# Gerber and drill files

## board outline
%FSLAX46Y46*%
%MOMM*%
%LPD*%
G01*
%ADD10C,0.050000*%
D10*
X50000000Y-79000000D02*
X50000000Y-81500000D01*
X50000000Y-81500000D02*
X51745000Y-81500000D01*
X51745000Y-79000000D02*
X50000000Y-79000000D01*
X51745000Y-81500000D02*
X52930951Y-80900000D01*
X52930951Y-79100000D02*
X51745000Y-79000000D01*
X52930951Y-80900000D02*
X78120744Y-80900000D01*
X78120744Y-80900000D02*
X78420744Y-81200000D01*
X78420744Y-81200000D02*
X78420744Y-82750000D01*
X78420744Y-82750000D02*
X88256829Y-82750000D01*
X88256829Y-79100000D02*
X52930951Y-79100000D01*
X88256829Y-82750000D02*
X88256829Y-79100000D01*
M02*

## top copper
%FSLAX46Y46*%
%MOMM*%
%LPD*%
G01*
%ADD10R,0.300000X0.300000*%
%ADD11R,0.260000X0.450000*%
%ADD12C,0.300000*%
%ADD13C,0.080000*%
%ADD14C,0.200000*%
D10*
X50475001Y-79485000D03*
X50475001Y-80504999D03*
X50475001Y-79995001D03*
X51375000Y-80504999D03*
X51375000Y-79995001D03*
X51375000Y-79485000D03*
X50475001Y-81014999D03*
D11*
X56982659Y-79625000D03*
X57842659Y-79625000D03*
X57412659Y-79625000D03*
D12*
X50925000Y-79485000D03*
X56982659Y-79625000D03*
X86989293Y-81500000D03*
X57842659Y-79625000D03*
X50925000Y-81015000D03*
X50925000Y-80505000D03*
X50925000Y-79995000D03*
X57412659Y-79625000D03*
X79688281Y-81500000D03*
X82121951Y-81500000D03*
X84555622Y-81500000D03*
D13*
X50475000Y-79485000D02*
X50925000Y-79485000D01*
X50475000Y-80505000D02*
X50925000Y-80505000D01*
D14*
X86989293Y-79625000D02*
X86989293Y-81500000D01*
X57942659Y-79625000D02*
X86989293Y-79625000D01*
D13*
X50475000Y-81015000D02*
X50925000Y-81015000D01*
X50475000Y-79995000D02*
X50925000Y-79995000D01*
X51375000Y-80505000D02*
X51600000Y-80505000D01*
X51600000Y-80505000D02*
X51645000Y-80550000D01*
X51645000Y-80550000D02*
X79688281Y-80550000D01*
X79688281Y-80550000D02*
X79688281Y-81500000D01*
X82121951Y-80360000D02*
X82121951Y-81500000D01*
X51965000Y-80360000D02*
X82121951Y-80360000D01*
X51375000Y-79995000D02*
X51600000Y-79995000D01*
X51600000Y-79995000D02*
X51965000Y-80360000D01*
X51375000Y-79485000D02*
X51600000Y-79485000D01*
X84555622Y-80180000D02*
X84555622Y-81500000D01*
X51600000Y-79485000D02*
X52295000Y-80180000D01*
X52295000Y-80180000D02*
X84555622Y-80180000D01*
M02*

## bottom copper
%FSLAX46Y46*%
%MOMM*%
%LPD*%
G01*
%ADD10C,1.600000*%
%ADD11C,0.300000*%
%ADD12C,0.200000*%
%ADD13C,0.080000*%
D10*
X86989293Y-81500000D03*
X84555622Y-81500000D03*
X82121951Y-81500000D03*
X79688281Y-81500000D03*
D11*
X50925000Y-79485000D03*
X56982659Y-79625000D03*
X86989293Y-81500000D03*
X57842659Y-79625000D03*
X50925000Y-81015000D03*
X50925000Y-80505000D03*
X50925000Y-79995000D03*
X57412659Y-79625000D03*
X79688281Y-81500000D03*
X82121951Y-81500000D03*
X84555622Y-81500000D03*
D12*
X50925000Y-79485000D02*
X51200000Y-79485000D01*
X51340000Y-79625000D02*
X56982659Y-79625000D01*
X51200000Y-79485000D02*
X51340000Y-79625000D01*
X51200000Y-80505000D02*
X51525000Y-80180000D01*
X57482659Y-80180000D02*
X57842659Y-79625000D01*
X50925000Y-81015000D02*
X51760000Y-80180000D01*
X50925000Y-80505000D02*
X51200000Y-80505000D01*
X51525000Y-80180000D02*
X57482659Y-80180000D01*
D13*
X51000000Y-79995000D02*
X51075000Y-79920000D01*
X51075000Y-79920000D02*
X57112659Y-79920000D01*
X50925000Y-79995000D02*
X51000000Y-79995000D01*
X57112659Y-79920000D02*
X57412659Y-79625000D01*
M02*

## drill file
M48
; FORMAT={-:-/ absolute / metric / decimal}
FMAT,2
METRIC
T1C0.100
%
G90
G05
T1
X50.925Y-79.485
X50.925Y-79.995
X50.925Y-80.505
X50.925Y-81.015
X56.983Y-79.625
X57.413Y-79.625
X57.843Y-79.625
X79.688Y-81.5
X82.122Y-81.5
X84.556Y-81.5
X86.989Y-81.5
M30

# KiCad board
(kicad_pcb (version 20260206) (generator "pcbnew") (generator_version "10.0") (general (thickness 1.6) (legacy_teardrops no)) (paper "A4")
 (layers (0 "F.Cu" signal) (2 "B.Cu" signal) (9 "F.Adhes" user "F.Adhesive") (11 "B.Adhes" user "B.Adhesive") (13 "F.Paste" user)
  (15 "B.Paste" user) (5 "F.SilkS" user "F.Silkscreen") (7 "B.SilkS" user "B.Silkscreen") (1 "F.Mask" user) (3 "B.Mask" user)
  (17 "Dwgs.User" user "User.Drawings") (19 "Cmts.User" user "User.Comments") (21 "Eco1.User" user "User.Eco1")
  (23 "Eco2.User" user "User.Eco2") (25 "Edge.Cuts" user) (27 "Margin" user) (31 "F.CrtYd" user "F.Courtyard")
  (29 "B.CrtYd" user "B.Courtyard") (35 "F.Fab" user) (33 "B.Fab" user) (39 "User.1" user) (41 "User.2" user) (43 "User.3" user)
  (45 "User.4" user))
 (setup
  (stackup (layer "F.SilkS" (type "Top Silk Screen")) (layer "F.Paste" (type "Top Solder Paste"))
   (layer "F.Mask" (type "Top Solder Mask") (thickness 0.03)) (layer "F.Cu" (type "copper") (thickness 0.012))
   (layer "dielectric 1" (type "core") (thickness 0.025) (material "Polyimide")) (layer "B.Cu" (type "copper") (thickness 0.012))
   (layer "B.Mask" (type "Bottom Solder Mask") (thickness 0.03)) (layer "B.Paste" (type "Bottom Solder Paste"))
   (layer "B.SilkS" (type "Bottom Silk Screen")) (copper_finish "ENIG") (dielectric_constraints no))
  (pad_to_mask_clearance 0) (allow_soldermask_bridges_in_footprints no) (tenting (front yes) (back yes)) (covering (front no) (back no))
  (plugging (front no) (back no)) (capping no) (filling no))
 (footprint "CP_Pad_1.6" (layer "F.Cu") (at 79.688281 81.5)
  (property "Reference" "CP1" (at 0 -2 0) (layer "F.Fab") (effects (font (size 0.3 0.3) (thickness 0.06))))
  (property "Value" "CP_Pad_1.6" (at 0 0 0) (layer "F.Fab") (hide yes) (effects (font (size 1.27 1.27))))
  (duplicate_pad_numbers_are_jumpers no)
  (pad "1" smd circle (at 0 0) (size 1.6 1.6) (layers "B.Cu" "B.Mask") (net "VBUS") (solder_mask_margin 0.1)))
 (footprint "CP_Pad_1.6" (layer "F.Cu") (at 86.989293 81.5)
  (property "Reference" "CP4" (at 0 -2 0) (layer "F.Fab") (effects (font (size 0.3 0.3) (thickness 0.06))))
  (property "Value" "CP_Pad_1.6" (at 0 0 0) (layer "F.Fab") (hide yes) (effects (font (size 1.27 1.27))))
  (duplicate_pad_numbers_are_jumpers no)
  (pad "1" smd circle (at 0 0) (size 1.6 1.6) (layers "B.Cu" "B.Mask") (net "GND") (solder_mask_margin 0.1)))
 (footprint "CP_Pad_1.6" (layer "F.Cu") (at 82.121951 81.5)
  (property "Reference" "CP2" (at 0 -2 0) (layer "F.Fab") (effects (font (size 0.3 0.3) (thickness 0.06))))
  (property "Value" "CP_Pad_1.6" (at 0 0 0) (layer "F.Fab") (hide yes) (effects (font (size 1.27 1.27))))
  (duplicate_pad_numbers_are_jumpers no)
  (pad "1" smd circle (at 0 0) (size 1.6 1.6) (layers "B.Cu" "B.Mask") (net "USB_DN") (solder_mask_margin 0.1)))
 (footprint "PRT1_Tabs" (layer "F.Cu") (at 57.412659 79.625)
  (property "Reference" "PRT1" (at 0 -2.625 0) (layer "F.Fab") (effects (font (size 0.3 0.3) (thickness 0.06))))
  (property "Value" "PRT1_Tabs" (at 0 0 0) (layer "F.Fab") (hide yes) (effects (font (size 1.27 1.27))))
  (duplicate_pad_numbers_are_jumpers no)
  (pad "1" smd rect (at -0.43 0) (size 0.26 0.45) (layers "F.Cu" "F.Mask") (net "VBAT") (solder_mask_margin 0.05) (thermal_bridge_angle 45))
  (pad "2" smd rect (at 0.43 0) (size 0.26 0.45) (layers "F.Cu" "F.Mask") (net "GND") (solder_mask_margin 0.05) (thermal_bridge_angle 45))
  (pad "3" smd rect (at 0 0) (size 0.26 0.45) (layers "F.Cu" "F.Mask") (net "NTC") (solder_mask_margin 0.05) (thermal_bridge_angle 45)))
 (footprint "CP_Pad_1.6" (layer "F.Cu") (at 84.555622 81.5)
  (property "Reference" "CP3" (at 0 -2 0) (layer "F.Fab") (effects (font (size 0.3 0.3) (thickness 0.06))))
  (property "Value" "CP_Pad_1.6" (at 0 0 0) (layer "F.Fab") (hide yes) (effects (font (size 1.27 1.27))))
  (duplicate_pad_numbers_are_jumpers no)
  (pad "1" smd circle (at 0 0) (size 1.6 1.6) (layers "B.Cu" "B.Mask") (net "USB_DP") (solder_mask_margin 0.1)))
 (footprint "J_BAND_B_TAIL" (layer "F.Cu") (at 50.9 80.25)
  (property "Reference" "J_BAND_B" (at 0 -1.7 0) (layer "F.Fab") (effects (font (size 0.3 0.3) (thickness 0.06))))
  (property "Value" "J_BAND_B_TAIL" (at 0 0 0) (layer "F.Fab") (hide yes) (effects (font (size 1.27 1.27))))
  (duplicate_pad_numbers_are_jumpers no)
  (pad "1" smd rect (at -0.424999 -0.765) (size 0.3 0.3) (layers "F.Cu" "F.Mask") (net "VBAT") (solder_mask_margin 0.05)
   (thermal_bridge_angle 45))
  (pad "2" smd rect (at -0.424999 0.254999) (size 0.3 0.3) (layers "F.Cu" "F.Mask") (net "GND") (solder_mask_margin 0.05)
   (thermal_bridge_angle 45))
  (pad "3" smd rect (at -0.424999 -0.254999) (size 0.3 0.3) (layers "F.Cu" "F.Mask") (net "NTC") (solder_mask_margin 0.05)
   (thermal_bridge_angle 45))
  (pad "4" smd rect (at 0.475 0.254999) (size 0.3 0.3) (layers "F.Cu" "F.Mask") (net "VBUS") (solder_mask_margin 0.05)
   (thermal_bridge_angle 45))
  (pad "5" smd rect (at 0.475 -0.254999) (size 0.3 0.3) (layers "F.Cu" "F.Mask") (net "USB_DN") (solder_mask_margin 0.05)
   (thermal_bridge_angle 45))
  (pad "6" smd rect (at 0.475 -0.765) (size 0.3 0.3) (layers "F.Cu" "F.Mask") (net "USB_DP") (solder_mask_margin 0.05)
   (thermal_bridge_angle 45))
  (pad "7" smd rect (at -0.424999 0.764999) (size 0.3 0.3) (layers "F.Cu" "F.Mask") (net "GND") (solder_mask_margin 0.05)
   (thermal_bridge_angle 45)))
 (gr_line (start 50 79) (end 50 81.5) (stroke (width 0.05) (type default)) (layer "Edge.Cuts"))
 (gr_line (start 50 81.5) (end 51.745 81.5) (stroke (width 0.05) (type default)) (layer "Edge.Cuts"))
 (gr_line (start 51.745 79) (end 50 79) (stroke (width 0.05) (type default)) (layer "Edge.Cuts"))
 (gr_line (start 51.745 81.5) (end 52.930951 80.9) (stroke (width 0.05) (type default)) (layer "Edge.Cuts"))
 (gr_line (start 52.930951 79.1) (end 51.745 79) (stroke (width 0.05) (type default)) (layer "Edge.Cuts"))
 (gr_line (start 52.930951 80.9) (end 78.120744 80.9) (stroke (width 0.05) (type default)) (layer "Edge.Cuts"))
 (gr_line (start 78.120744 80.9) (end 78.420744 81.2) (stroke (width 0.05) (type default)) (layer "Edge.Cuts"))
 (gr_line (start 78.420744 81.2) (end 78.420744 82.75) (stroke (width 0.05) (type default)) (layer "Edge.Cuts"))
 (gr_line (start 78.420744 82.75) (end 88.256829 82.75) (stroke (width 0.05) (type default)) (layer "Edge.Cuts"))
 (gr_line (start 88.256829 79.1) (end 52.930951 79.1) (stroke (width 0.05) (type default)) (layer "Edge.Cuts"))
 (gr_line (start 88.256829 82.75) (end 88.256829 79.1) (stroke (width 0.05) (type default)) (layer "Edge.Cuts"))
 (segment (start 50.475 79.485) (end 50.925 79.485) (width 0.08) (layer "F.Cu") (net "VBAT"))
 (via (at 50.925 79.485) (size 0.3) (drill 0.1) (layers "F.Cu" "B.Cu") (tenting (front yes) (back yes)) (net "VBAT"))
 (via (at 56.982659 79.625) (size 0.3) (drill 0.1) (layers "F.Cu" "B.Cu") (tenting (front yes) (back yes)) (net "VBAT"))
 (segment (start 51.2 79.485) (end 51.34 79.625) (width 0.2) (layer "B.Cu") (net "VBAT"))
 (segment (start 51.34 79.625) (end 56.982659 79.625) (width 0.2) (layer "B.Cu") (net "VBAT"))
 (segment (start 50.925 79.485) (end 51.2 79.485) (width 0.2) (layer "B.Cu") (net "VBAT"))
 (segment (start 57.942659 79.625) (end 86.989293 79.625) (width 0.2) (layer "F.Cu") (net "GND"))
 (segment (start 50.475 81.015) (end 50.925 81.015) (width 0.08) (layer "F.Cu") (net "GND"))
 (segment (start 86.989293 79.625) (end 86.989293 81.5) (width 0.2) (layer "F.Cu") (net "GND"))
 (segment (start 50.475 80.505) (end 50.925 80.505) (width 0.08) (layer "F.Cu") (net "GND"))
 (via (at 50.925 80.505) (size 0.3) (drill 0.1) (layers "F.Cu" "B.Cu") (tenting (front yes) (back yes)) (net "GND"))
 (via (at 50.925 81.015) (size 0.3) (drill 0.1) (layers "F.Cu" "B.Cu") (tenting (front yes) (back yes)) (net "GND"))
 (via (at 57.842659 79.625) (size 0.3) (drill 0.1) (layers "F.Cu" "B.Cu") (tenting (front yes) (back yes)) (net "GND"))
 (via (at 86.989293 81.5) (size 0.3) (drill 0.1) (layers "F.Cu" "B.Cu") (tenting (front yes) (back yes)) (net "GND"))
 (segment (start 50.925 81.015) (end 51.76 80.18) (width 0.2) (layer "B.Cu") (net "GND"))
 (segment (start 51.525 80.18) (end 57.482659 80.18) (width 0.2) (layer "B.Cu") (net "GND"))
 (segment (start 57.482659 80.18) (end 57.842659 79.625) (width 0.2) (layer "B.Cu") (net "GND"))
 (segment (start 51.2 80.505) (end 51.525 80.18) (width 0.2) (layer "B.Cu") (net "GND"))
 (segment (start 50.925 80.505) (end 51.2 80.505) (width 0.2) (layer "B.Cu") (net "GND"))
 (segment (start 50.475 79.995) (end 50.925 79.995) (width 0.08) (layer "F.Cu") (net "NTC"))
 (via (at 50.925 79.995) (size 0.3) (drill 0.1) (layers "F.Cu" "B.Cu") (tenting (front yes) (back yes)) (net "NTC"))
 (via (at 57.412659 79.625) (size 0.3) (drill 0.1) (layers "F.Cu" "B.Cu") (tenting (front yes) (back yes)) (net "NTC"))
 (segment (start 51.075 79.92) (end 57.112659 79.92) (width 0.08) (layer "B.Cu") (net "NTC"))
 (segment (start 50.925 79.995) (end 51 79.995) (width 0.08) (layer "B.Cu") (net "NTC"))
 (segment (start 57.112659 79.92) (end 57.412659 79.625) (width 0.08) (layer "B.Cu") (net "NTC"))
 (segment (start 51 79.995) (end 51.075 79.92) (width 0.08) (layer "B.Cu") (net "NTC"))
 (segment (start 51.6 80.505) (end 51.645 80.55) (width 0.08) (layer "F.Cu") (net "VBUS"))
 (segment (start 79.688281 80.55) (end 79.688281 81.5) (width 0.08) (layer "F.Cu") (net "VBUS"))
 (segment (start 51.375 80.505) (end 51.6 80.505) (width 0.08) (layer "F.Cu") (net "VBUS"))
 (segment (start 51.645 80.55) (end 79.688281 80.55) (width 0.08) (layer "F.Cu") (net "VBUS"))
 (via (at 79.688281 81.5) (size 0.3) (drill 0.1) (layers "F.Cu" "B.Cu") (tenting (front yes) (back yes)) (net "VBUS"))
 (segment (start 51.6 79.995) (end 51.965 80.36) (width 0.08) (layer "F.Cu") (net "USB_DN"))
 (segment (start 51.965 80.36) (end 82.121951 80.36) (width 0.08) (layer "F.Cu") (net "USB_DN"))
 (segment (start 51.375 79.995) (end 51.6 79.995) (width 0.08) (layer "F.Cu") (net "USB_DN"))
 (segment (start 82.121951 80.36) (end 82.121951 81.5) (width 0.08) (layer "F.Cu") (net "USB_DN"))
 (via (at 82.121951 81.5) (size 0.3) (drill 0.1) (layers "F.Cu" "B.Cu") (tenting (front yes) (back yes)) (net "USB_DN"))
 (segment (start 52.295 80.18) (end 84.555622 80.18) (width 0.08) (layer "F.Cu") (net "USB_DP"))
 (segment (start 51.375 79.485) (end 51.6 79.485) (width 0.08) (layer "F.Cu") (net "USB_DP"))
 (segment (start 51.6 79.485) (end 52.295 80.18) (width 0.08) (layer "F.Cu") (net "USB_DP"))
 (segment (start 84.555622 80.18) (end 84.555622 81.5) (width 0.08) (layer "F.Cu") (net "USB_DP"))
 (via (at 84.555622 81.5) (size 0.3) (drill 0.1) (layers "F.Cu" "B.Cu") (tenting (front yes) (back yes)) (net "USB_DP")))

